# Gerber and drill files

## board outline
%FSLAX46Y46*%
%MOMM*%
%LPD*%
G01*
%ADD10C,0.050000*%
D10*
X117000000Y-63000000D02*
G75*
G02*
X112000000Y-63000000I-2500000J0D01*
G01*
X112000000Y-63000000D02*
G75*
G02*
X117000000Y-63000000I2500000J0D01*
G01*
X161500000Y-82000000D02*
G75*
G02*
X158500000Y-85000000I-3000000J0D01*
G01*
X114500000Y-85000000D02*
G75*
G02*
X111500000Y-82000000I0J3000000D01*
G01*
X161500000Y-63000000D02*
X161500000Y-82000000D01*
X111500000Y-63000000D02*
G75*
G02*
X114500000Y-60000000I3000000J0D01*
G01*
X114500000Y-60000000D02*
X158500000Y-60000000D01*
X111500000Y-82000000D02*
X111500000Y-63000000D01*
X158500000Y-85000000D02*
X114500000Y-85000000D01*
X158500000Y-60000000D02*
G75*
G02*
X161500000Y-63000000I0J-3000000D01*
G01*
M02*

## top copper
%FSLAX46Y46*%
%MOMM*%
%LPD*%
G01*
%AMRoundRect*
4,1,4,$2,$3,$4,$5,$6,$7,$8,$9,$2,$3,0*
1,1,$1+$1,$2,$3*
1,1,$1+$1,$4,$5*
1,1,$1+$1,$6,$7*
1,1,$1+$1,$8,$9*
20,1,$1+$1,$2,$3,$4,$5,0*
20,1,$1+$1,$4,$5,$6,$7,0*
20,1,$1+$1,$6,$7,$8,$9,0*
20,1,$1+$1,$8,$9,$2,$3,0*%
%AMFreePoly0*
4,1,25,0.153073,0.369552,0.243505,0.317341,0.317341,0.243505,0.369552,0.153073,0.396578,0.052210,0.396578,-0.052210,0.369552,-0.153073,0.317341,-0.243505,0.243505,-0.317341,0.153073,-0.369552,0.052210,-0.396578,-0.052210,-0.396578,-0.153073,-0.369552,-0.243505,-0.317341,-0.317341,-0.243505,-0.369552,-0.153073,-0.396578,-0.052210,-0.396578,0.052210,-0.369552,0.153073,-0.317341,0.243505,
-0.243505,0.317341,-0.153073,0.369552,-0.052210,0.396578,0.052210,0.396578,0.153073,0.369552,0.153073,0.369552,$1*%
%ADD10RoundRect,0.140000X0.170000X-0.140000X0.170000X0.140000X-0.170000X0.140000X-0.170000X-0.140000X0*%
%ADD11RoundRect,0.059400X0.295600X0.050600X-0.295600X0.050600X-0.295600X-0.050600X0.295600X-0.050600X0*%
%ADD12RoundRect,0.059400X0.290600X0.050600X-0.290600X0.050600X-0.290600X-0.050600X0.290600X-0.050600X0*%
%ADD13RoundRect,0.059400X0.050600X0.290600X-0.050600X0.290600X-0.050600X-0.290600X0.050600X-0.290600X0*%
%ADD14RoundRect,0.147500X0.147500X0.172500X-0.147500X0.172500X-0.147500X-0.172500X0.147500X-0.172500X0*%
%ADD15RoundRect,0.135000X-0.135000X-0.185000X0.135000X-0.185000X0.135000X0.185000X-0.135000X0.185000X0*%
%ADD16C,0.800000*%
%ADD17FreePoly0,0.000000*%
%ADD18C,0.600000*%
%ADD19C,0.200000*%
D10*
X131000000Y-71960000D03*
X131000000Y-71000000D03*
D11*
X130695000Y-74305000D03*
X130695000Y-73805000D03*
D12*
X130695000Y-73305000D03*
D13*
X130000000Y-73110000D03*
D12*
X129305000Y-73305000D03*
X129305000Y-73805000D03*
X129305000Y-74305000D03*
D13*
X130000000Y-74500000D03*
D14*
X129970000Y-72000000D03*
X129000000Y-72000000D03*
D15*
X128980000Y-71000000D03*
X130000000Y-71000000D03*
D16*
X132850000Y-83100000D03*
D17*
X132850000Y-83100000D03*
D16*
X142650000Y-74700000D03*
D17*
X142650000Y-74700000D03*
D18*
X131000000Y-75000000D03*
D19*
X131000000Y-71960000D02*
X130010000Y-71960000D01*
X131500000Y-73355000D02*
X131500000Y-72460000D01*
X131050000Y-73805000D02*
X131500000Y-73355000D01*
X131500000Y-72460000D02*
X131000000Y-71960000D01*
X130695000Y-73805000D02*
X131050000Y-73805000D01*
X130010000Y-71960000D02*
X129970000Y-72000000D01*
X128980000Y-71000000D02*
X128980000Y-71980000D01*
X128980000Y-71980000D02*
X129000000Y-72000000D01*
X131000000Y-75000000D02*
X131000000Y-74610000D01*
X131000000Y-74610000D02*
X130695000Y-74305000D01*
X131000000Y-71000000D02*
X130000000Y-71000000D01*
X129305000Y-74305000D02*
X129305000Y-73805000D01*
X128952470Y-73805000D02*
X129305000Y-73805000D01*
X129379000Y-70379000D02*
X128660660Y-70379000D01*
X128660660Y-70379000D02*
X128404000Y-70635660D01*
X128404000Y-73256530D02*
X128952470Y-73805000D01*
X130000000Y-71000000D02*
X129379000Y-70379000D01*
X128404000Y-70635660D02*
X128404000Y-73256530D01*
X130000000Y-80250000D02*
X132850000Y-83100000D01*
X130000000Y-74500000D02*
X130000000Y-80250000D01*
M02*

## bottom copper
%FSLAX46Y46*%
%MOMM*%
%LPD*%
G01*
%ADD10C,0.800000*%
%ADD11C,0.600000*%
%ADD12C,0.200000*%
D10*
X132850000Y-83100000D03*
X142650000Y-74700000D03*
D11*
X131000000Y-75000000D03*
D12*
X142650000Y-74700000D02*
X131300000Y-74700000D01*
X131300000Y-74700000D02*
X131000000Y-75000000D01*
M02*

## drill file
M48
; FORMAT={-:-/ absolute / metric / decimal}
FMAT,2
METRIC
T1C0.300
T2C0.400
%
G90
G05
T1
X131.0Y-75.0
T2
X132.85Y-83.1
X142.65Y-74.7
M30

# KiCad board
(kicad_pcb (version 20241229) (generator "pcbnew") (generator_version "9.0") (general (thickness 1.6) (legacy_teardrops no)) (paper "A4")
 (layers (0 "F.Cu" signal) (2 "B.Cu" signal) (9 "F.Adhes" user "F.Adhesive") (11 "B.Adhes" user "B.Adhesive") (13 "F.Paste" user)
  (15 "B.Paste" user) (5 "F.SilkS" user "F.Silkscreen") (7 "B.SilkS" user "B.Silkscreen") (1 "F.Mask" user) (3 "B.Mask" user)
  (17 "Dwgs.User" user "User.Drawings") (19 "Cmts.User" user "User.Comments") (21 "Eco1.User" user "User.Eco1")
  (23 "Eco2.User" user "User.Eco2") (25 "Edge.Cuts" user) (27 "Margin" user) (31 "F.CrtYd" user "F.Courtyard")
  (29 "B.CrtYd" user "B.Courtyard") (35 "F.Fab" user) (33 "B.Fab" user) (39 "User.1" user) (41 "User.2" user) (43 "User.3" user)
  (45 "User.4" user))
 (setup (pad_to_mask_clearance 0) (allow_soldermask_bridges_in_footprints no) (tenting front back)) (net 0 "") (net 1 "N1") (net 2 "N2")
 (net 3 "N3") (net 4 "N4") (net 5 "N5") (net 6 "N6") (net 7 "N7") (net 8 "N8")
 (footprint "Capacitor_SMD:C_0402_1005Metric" (layer "F.Cu") (at 131 71.48 90)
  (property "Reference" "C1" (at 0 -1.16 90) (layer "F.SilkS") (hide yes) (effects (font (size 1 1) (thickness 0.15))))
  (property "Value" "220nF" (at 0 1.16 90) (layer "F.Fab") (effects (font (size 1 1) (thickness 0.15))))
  (pad "1" smd roundrect (at -0.48 0 90) (size 0.56 0.62) (layers "F.Cu" "F.Mask" "F.Paste") (roundrect_rratio 0.25) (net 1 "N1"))
  (pad "2" smd roundrect (at 0.48 0 90) (size 0.56 0.62) (layers "F.Cu" "F.Mask" "F.Paste") (roundrect_rratio 0.25) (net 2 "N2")))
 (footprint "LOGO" (layer "F.Cu") (at 144.573999 73.00007)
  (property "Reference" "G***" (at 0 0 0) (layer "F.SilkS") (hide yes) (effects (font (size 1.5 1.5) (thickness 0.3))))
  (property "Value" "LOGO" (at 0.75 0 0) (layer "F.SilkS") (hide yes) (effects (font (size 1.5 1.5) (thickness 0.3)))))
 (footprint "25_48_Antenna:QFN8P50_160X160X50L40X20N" (layer "F.Cu") (at 130 73.805 180)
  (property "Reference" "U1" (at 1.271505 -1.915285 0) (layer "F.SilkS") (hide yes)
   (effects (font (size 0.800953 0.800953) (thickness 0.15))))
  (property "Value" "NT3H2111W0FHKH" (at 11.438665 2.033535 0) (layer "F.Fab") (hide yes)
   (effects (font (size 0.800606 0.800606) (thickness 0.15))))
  (pad "1" smd roundrect (at -0.695 -0.5 180) (size 0.71 0.22) (layers "F.Cu" "F.Mask" "F.Paste") (roundrect_rratio 0.27) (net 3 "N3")
   (solder_mask_margin 0.102))
  (pad "2" smd roundrect (at -0.695 0 180) (size 0.71 0.22) (layers "F.Cu" "F.Mask" "F.Paste") (roundrect_rratio 0.27) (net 1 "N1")
   (solder_mask_margin 0.102))
  (pad "3" smd roundrect (at -0.695 0.5 180) (size 0.7 0.22) (layers "F.Cu" "F.Mask" "F.Paste") (roundrect_rratio 0.27) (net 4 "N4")
   (solder_mask_margin 0.102))
  (pad "4" smd roundrect (at 0 0.695 180) (size 0.22 0.7) (layers "F.Cu" "F.Mask" "F.Paste") (roundrect_rratio 0.27) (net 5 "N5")
   (solder_mask_margin 0.102))
  (pad "5" smd roundrect (at 0.695 0.5 180) (size 0.7 0.22) (layers "F.Cu" "F.Mask" "F.Paste") (roundrect_rratio 0.27) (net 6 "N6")
   (solder_mask_margin 0.102))
  (pad "6" smd roundrect (at 0.695 0 180) (size 0.7 0.22) (layers "F.Cu" "F.Mask" "F.Paste") (roundrect_rratio 0.27) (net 2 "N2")
   (solder_mask_margin 0.102))
  (pad "7" smd roundrect (at 0.695 -0.5 180) (size 0.7 0.22) (layers "F.Cu" "F.Mask" "F.Paste") (roundrect_rratio 0.27) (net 2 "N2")
   (solder_mask_margin 0.102))
  (pad "8" smd roundrect (at 0 -0.695 180) (size 0.22 0.7) (layers "F.Cu" "F.Mask" "F.Paste") (roundrect_rratio 0.27) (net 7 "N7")
   (solder_mask_margin 0.102)))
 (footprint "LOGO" (layer "F.Cu") (at 114.5 76)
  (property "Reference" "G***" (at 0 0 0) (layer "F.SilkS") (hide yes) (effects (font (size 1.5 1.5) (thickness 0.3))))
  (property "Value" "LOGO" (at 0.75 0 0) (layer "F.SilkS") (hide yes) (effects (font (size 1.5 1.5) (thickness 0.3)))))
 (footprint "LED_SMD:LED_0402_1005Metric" (layer "F.Cu") (at 129.485 72 180)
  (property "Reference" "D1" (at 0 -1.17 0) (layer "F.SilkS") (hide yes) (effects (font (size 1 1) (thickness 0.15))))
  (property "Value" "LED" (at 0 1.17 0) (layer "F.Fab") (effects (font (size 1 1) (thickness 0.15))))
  (pad "1" smd roundrect (at -0.485 0 180) (size 0.59 0.64) (layers "F.Cu" "F.Mask" "F.Paste") (roundrect_rratio 0.25) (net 1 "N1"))
  (pad "2" smd roundrect (at 0.485 0 180) (size 0.59 0.64) (layers "F.Cu" "F.Mask" "F.Paste") (roundrect_rratio 0.25) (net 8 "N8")))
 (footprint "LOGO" (layer "F.Cu") (at 114.5 81.5)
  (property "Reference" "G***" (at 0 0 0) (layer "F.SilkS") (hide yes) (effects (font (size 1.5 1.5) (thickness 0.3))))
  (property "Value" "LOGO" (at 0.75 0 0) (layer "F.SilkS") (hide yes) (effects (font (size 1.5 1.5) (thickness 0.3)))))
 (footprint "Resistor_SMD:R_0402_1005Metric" (layer "F.Cu") (at 129.49 71)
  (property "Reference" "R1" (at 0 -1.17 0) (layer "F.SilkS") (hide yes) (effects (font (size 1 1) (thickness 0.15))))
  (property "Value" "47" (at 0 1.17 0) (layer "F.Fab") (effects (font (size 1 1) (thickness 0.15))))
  (pad "1" smd roundrect (at -0.51 0) (size 0.54 0.64) (layers "F.Cu" "F.Mask" "F.Paste") (roundrect_rratio 0.25) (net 8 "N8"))
  (pad "2" smd roundrect (at 0.51 0) (size 0.54 0.64) (layers "F.Cu" "F.Mask" "F.Paste") (roundrect_rratio 0.25) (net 2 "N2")))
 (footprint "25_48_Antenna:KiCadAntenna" (layer "F.Cu") (at 132.45 61.5)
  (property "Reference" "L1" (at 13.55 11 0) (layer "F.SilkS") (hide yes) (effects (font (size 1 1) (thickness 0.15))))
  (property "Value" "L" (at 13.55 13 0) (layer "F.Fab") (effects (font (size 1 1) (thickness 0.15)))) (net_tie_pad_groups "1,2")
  (pad "1" thru_hole circle (at 0.4 21.6) (size 0.8 0.8) (drill 0.4) (layers "*.Cu" "*.Mask") (remove_unused_layers no) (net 7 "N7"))
  (pad "1" smd custom (at 0.4 21.6) (size 0.8 0.8) (layers "F.Cu") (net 7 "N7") (zone_connect 0) (thermal_bridge_angle 90)
   (options (clearance outline) (anchor circle)) (primitives))
  (pad "2" thru_hole circle (at 10.2 13.2) (size 0.8 0.8) (drill 0.4) (layers "*.Cu" "*.Mask") (remove_unused_layers no) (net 3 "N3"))
  (pad "2" smd custom (at 10.2 13.2) (size 0.8 0.8) (layers "F.Cu") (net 3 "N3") (zone_connect 0) (thermal_bridge_angle 90)
   (options (clearance outline) (anchor circle)) (primitives)))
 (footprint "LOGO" (layer "F.Cu") (at 124 74.5)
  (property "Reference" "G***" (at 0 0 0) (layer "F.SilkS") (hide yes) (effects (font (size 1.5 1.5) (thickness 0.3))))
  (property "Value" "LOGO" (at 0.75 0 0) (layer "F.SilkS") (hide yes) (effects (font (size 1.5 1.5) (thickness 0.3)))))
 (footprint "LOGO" (layer "B.Cu") (at 146.5 73)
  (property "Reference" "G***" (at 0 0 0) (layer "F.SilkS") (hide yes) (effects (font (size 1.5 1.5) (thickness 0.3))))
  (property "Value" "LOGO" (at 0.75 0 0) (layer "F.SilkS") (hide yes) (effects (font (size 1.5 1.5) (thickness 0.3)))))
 (gr_circle (center 114.5 63) (end 114.5 60.5) (stroke (width 0.05) (type default)) (fill no) (layer "Edge.Cuts"))
 (gr_arc (start 161.5 82) (mid 160.62132 84.12132) (end 158.5 85) (stroke (width 0.05) (type default)) (layer "Edge.Cuts"))
 (gr_arc (start 114.5 85) (mid 112.37868 84.12132) (end 111.5 82) (stroke (width 0.05) (type default)) (layer "Edge.Cuts"))
 (gr_line (start 161.5 63) (end 161.5 82) (stroke (width 0.05) (type default)) (layer "Edge.Cuts"))
 (gr_arc (start 111.5 63) (mid 112.37868 60.87868) (end 114.5 60) (stroke (width 0.05) (type default)) (layer "Edge.Cuts"))
 (gr_line (start 114.5 60) (end 158.5 60) (stroke (width 0.05) (type default)) (layer "Edge.Cuts"))
 (gr_line (start 111.5 82) (end 111.5 63) (stroke (width 0.05) (type default)) (layer "Edge.Cuts"))
 (gr_line (start 158.5 85) (end 114.5 85) (stroke (width 0.05) (type default)) (layer "Edge.Cuts"))
 (gr_arc (start 158.5 60) (mid 160.62132 60.87868) (end 161.5 63) (stroke (width 0.05) (type default)) (layer "Edge.Cuts"))
 (segment (start 131 71.96) (end 130.01 71.96) (width 0.2) (layer "F.Cu") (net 1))
 (segment (start 131.5 73.355) (end 131.5 72.46) (width 0.2) (layer "F.Cu") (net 1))
 (segment (start 131.05 73.805) (end 131.5 73.355) (width 0.2) (layer "F.Cu") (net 1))
 (segment (start 131.5 72.46) (end 131 71.96) (width 0.2) (layer "F.Cu") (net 1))
 (segment (start 130.695 73.805) (end 131.05 73.805) (width 0.2) (layer "F.Cu") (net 1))
 (segment (start 130.01 71.96) (end 129.97 72) (width 0.2) (layer "F.Cu") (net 1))
 (segment (start 128.98 71) (end 128.98 71.98) (width 0.2) (layer "F.Cu") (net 8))
 (segment (start 128.98 71.98) (end 129 72) (width 0.2) (layer "F.Cu") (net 8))
 (segment (start 131 75) (end 131 74.61) (width 0.2) (layer "F.Cu") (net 3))
 (segment (start 131 74.61) (end 130.695 74.305) (width 0.2) (layer "F.Cu") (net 3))
 (via (at 131 75) (size 0.6) (drill 0.3) (layers "F.Cu" "B.Cu") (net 3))
 (segment (start 142.65 74.7) (end 131.3 74.7) (width 0.2) (layer "B.Cu") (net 3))
 (segment (start 131.3 74.7) (end 131 75) (width 0.2) (layer "B.Cu") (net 3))
 (segment (start 131 71) (end 130 71) (width 0.2) (layer "F.Cu") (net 2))
 (segment (start 129.305 74.305) (end 129.305 73.805) (width 0.2) (layer "F.Cu") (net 2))
 (segment (start 128.95247 73.805) (end 129.305 73.805) (width 0.2) (layer "F.Cu") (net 2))
 (segment (start 129.379 70.379) (end 128.66066 70.379) (width 0.2) (layer "F.Cu") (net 2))
 (segment (start 128.66066 70.379) (end 128.404 70.63566) (width 0.2) (layer "F.Cu") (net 2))
 (segment (start 128.404 73.25653) (end 128.95247 73.805) (width 0.2) (layer "F.Cu") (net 2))
 (segment (start 130 71) (end 129.379 70.379) (width 0.2) (layer "F.Cu") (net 2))
 (segment (start 128.404 70.63566) (end 128.404 73.25653) (width 0.2) (layer "F.Cu") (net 2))
 (segment (start 130 80.25) (end 132.85 83.1) (width 0.2) (layer "F.Cu") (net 7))
 (segment (start 130 74.5) (end 130 80.25) (width 0.2) (layer "F.Cu") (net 7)))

